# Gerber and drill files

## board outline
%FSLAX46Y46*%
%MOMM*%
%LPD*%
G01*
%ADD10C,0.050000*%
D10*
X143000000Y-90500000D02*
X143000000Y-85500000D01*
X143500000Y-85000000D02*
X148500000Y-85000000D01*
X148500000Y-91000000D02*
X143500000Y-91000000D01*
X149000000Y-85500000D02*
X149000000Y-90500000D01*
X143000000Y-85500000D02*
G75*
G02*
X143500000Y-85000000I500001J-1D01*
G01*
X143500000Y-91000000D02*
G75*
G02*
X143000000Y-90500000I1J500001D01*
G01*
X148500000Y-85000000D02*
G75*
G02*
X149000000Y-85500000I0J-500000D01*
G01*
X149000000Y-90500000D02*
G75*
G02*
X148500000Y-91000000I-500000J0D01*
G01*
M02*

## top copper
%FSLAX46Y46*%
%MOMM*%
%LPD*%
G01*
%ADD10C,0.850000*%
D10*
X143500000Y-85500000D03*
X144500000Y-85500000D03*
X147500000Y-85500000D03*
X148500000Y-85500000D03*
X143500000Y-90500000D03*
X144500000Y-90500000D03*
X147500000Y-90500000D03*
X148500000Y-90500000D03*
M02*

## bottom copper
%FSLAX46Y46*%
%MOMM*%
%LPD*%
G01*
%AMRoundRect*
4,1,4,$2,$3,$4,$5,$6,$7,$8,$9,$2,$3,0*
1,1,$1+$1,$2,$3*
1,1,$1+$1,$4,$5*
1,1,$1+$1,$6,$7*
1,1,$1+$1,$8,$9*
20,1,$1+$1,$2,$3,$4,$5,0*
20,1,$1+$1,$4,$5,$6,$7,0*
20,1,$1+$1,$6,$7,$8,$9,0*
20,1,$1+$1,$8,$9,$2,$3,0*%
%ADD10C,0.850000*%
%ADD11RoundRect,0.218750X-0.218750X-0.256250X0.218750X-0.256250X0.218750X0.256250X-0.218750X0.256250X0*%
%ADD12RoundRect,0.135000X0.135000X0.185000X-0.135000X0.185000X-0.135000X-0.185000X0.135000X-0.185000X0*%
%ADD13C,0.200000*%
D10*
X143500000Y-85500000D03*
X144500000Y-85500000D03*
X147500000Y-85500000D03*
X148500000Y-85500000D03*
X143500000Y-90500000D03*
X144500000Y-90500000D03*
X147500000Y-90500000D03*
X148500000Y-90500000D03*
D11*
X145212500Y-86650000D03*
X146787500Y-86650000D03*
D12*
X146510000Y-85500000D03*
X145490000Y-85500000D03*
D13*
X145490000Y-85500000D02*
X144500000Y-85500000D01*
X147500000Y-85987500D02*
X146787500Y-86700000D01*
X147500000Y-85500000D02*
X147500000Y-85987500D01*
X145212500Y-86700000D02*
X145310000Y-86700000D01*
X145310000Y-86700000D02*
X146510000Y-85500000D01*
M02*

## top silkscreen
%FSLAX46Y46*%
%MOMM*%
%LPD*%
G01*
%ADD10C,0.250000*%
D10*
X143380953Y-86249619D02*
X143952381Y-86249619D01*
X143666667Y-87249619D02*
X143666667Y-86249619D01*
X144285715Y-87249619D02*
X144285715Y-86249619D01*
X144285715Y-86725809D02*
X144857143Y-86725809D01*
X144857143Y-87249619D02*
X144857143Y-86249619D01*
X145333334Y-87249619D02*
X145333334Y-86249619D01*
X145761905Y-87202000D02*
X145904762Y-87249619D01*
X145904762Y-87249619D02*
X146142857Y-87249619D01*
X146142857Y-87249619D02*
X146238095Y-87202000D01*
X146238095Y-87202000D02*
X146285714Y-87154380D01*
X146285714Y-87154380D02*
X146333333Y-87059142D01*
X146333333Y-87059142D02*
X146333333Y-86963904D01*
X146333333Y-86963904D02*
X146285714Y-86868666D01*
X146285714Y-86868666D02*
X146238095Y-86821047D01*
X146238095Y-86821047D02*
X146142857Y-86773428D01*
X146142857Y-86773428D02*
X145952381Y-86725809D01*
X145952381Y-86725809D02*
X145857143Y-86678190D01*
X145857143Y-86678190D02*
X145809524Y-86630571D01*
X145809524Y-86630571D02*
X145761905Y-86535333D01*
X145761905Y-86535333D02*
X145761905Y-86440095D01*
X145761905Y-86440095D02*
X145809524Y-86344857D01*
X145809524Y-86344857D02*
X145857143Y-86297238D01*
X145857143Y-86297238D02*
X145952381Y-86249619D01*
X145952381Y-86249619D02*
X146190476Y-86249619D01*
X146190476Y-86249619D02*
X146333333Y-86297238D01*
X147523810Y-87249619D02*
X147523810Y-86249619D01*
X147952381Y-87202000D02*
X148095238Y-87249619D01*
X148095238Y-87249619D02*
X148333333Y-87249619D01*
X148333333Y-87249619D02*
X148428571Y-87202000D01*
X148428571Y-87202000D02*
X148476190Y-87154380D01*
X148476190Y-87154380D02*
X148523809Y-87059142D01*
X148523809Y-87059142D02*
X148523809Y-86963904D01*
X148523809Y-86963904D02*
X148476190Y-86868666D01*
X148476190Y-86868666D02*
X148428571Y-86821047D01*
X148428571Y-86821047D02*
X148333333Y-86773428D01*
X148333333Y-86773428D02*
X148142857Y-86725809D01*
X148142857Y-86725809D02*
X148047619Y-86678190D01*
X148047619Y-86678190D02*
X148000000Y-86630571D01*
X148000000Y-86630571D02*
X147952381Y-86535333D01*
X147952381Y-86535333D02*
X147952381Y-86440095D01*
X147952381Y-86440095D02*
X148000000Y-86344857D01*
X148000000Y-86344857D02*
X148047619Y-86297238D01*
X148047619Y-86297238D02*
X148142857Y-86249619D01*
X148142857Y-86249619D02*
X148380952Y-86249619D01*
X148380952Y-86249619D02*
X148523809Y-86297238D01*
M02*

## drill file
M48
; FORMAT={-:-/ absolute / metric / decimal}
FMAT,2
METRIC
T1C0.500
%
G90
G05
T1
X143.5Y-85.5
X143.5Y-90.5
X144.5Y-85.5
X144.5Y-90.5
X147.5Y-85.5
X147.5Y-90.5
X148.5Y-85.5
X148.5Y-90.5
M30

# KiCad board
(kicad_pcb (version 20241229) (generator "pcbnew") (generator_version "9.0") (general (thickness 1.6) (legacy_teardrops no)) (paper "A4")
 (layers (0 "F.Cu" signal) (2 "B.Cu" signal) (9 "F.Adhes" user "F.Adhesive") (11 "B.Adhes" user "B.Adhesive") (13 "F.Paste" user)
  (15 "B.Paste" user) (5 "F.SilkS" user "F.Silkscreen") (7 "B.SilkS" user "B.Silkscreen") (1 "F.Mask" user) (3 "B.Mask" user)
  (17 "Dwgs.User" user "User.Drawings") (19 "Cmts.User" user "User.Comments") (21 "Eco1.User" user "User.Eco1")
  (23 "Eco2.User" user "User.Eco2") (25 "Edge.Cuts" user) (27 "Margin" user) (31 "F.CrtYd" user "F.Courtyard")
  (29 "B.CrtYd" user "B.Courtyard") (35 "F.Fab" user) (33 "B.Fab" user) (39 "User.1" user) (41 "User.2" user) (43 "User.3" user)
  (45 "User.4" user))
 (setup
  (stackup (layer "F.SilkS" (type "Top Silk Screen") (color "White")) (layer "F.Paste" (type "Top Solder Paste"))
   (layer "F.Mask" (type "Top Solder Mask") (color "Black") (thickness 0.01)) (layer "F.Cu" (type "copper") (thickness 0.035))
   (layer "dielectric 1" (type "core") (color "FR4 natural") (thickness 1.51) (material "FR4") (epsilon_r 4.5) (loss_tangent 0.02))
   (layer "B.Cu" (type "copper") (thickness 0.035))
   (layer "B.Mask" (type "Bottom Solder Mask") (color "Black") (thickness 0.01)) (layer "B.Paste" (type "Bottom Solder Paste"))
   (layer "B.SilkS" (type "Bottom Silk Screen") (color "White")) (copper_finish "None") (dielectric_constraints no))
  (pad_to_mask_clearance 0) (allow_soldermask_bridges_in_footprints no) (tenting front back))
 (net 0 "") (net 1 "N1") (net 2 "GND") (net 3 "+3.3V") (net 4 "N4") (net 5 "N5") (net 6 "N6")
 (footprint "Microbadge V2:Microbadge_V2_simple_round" (layer "F.Cu") (at 146 88)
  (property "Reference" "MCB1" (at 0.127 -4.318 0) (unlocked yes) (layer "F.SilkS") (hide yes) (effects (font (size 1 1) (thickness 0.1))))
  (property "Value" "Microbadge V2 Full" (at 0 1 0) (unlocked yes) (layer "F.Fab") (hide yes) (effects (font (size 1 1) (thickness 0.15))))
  (fp_line (start -3 2.5) (end -3 -2.5) (stroke (width 0.05) (type default)) (layer "Edge.Cuts"))
  (fp_line (start -2.5 -3) (end 2.5 -3) (stroke (width 0.05) (type default)) (layer "Edge.Cuts"))
  (fp_line (start 2.5 3) (end -2.5 3) (stroke (width 0.05) (type default)) (layer "Edge.Cuts"))
  (fp_line (start 3 -2.5) (end 3 2.5) (stroke (width 0.05) (type default)) (layer "Edge.Cuts"))
  (fp_arc (start -3 -2.5) (mid -2.853553 -2.853553) (end -2.5 -3) (stroke (width 0.05) (type default)) (layer "Edge.Cuts"))
  (fp_arc (start -2.5 3) (mid -2.853553 2.853553) (end -3 2.5) (stroke (width 0.05) (type default)) (layer "Edge.Cuts"))
  (fp_arc (start 2.5 -3) (mid 2.853553 -2.853553) (end 3 -2.5) (stroke (width 0.05) (type default)) (layer "Edge.Cuts"))
  (fp_arc (start 3 2.5) (mid 2.853553 2.853553) (end 2.5 3) (stroke (width 0.05) (type default)) (layer "Edge.Cuts"))
  (pad "1" thru_hole circle (at -2.5 -2.5 90) (size 0.85 0.85) (drill 0.5) (layers "*.Cu" "*.Mask") (remove_unused_layers no) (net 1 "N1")
   (thermal_bridge_angle 90))
  (pad "2" thru_hole circle (at -1.5 -2.5 90) (size 0.85 0.85) (drill 0.5) (layers "*.Cu" "*.Mask") (remove_unused_layers no) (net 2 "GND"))
  (pad "5" thru_hole circle (at 1.5 -2.5 90) (size 0.85 0.85) (drill 0.5) (layers "*.Cu" "*.Mask") (remove_unused_layers no) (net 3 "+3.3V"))
  (pad "6" thru_hole circle (at 2.5 -2.5 90) (size 0.85 0.85) (drill 0.5) (layers "*.Cu" "*.Mask") (remove_unused_layers no) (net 2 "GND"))
  (pad "7" thru_hole circle (at -2.5 2.5 90) (size 0.85 0.85) (drill 0.5) (layers "*.Cu" "*.Mask") (remove_unused_layers no) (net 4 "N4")
   (thermal_bridge_angle 90))
  (pad "8" thru_hole circle (at -1.5 2.5 90) (size 0.85 0.85) (drill 0.5) (layers "*.Cu" "*.Mask") (remove_unused_layers no) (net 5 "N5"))
  (pad "11" thru_hole circle (at 1.5 2.5 90) (size 0.85 0.85) (drill 0.5) (layers "*.Cu" "*.Mask") (remove_unused_layers no) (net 3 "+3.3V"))
  (pad "12" thru_hole circle (at 2.5 2.5 90) (size 0.85 0.85) (drill 0.5) (layers "*.Cu" "*.Mask") (remove_unused_layers no) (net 2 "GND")))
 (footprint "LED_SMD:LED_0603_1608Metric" (layer "B.Cu") (at 146 86.65)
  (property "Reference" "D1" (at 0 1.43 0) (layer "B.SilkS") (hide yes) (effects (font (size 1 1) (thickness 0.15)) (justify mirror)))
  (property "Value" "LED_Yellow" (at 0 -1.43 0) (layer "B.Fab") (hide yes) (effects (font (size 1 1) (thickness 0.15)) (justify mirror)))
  (pad "1" smd roundrect (at -0.7875 0) (size 0.875 0.95) (layers "B.Cu" "B.Mask" "B.Paste") (roundrect_rratio 0.25) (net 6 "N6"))
  (pad "2" smd roundrect (at 0.7875 0) (size 0.875 0.95) (layers "B.Cu" "B.Mask" "B.Paste") (roundrect_rratio 0.25) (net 3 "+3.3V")))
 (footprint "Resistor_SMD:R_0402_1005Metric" (layer "B.Cu") (at 146 85.5 180)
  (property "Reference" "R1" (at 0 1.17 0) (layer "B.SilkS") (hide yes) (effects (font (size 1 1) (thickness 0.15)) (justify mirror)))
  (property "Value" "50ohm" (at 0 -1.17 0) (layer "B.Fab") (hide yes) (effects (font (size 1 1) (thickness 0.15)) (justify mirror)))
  (pad "1" smd roundrect (at -0.51 0 180) (size 0.54 0.64) (layers "B.Cu" "B.Mask" "B.Paste") (roundrect_rratio 0.25) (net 6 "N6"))
  (pad "2" smd roundrect (at 0.51 0 180) (size 0.54 0.64) (layers "B.Cu" "B.Mask" "B.Paste") (roundrect_rratio 0.25) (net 2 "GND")))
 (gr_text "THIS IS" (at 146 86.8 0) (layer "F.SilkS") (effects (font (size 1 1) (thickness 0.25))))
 (segment (start 145.49 85.5) (end 144.5 85.5) (width 0.2) (layer "B.Cu") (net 2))
 (segment (start 147.5 85.9875) (end 146.7875 86.7) (width 0.2) (layer "B.Cu") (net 3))
 (segment (start 147.5 85.5) (end 147.5 85.9875) (width 0.2) (layer "B.Cu") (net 3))
 (segment (start 145.2125 86.7) (end 145.31 86.7) (width 0.2) (layer "B.Cu") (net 6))
 (segment (start 145.31 86.7) (end 146.51 85.5) (width 0.2) (layer "B.Cu") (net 6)))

